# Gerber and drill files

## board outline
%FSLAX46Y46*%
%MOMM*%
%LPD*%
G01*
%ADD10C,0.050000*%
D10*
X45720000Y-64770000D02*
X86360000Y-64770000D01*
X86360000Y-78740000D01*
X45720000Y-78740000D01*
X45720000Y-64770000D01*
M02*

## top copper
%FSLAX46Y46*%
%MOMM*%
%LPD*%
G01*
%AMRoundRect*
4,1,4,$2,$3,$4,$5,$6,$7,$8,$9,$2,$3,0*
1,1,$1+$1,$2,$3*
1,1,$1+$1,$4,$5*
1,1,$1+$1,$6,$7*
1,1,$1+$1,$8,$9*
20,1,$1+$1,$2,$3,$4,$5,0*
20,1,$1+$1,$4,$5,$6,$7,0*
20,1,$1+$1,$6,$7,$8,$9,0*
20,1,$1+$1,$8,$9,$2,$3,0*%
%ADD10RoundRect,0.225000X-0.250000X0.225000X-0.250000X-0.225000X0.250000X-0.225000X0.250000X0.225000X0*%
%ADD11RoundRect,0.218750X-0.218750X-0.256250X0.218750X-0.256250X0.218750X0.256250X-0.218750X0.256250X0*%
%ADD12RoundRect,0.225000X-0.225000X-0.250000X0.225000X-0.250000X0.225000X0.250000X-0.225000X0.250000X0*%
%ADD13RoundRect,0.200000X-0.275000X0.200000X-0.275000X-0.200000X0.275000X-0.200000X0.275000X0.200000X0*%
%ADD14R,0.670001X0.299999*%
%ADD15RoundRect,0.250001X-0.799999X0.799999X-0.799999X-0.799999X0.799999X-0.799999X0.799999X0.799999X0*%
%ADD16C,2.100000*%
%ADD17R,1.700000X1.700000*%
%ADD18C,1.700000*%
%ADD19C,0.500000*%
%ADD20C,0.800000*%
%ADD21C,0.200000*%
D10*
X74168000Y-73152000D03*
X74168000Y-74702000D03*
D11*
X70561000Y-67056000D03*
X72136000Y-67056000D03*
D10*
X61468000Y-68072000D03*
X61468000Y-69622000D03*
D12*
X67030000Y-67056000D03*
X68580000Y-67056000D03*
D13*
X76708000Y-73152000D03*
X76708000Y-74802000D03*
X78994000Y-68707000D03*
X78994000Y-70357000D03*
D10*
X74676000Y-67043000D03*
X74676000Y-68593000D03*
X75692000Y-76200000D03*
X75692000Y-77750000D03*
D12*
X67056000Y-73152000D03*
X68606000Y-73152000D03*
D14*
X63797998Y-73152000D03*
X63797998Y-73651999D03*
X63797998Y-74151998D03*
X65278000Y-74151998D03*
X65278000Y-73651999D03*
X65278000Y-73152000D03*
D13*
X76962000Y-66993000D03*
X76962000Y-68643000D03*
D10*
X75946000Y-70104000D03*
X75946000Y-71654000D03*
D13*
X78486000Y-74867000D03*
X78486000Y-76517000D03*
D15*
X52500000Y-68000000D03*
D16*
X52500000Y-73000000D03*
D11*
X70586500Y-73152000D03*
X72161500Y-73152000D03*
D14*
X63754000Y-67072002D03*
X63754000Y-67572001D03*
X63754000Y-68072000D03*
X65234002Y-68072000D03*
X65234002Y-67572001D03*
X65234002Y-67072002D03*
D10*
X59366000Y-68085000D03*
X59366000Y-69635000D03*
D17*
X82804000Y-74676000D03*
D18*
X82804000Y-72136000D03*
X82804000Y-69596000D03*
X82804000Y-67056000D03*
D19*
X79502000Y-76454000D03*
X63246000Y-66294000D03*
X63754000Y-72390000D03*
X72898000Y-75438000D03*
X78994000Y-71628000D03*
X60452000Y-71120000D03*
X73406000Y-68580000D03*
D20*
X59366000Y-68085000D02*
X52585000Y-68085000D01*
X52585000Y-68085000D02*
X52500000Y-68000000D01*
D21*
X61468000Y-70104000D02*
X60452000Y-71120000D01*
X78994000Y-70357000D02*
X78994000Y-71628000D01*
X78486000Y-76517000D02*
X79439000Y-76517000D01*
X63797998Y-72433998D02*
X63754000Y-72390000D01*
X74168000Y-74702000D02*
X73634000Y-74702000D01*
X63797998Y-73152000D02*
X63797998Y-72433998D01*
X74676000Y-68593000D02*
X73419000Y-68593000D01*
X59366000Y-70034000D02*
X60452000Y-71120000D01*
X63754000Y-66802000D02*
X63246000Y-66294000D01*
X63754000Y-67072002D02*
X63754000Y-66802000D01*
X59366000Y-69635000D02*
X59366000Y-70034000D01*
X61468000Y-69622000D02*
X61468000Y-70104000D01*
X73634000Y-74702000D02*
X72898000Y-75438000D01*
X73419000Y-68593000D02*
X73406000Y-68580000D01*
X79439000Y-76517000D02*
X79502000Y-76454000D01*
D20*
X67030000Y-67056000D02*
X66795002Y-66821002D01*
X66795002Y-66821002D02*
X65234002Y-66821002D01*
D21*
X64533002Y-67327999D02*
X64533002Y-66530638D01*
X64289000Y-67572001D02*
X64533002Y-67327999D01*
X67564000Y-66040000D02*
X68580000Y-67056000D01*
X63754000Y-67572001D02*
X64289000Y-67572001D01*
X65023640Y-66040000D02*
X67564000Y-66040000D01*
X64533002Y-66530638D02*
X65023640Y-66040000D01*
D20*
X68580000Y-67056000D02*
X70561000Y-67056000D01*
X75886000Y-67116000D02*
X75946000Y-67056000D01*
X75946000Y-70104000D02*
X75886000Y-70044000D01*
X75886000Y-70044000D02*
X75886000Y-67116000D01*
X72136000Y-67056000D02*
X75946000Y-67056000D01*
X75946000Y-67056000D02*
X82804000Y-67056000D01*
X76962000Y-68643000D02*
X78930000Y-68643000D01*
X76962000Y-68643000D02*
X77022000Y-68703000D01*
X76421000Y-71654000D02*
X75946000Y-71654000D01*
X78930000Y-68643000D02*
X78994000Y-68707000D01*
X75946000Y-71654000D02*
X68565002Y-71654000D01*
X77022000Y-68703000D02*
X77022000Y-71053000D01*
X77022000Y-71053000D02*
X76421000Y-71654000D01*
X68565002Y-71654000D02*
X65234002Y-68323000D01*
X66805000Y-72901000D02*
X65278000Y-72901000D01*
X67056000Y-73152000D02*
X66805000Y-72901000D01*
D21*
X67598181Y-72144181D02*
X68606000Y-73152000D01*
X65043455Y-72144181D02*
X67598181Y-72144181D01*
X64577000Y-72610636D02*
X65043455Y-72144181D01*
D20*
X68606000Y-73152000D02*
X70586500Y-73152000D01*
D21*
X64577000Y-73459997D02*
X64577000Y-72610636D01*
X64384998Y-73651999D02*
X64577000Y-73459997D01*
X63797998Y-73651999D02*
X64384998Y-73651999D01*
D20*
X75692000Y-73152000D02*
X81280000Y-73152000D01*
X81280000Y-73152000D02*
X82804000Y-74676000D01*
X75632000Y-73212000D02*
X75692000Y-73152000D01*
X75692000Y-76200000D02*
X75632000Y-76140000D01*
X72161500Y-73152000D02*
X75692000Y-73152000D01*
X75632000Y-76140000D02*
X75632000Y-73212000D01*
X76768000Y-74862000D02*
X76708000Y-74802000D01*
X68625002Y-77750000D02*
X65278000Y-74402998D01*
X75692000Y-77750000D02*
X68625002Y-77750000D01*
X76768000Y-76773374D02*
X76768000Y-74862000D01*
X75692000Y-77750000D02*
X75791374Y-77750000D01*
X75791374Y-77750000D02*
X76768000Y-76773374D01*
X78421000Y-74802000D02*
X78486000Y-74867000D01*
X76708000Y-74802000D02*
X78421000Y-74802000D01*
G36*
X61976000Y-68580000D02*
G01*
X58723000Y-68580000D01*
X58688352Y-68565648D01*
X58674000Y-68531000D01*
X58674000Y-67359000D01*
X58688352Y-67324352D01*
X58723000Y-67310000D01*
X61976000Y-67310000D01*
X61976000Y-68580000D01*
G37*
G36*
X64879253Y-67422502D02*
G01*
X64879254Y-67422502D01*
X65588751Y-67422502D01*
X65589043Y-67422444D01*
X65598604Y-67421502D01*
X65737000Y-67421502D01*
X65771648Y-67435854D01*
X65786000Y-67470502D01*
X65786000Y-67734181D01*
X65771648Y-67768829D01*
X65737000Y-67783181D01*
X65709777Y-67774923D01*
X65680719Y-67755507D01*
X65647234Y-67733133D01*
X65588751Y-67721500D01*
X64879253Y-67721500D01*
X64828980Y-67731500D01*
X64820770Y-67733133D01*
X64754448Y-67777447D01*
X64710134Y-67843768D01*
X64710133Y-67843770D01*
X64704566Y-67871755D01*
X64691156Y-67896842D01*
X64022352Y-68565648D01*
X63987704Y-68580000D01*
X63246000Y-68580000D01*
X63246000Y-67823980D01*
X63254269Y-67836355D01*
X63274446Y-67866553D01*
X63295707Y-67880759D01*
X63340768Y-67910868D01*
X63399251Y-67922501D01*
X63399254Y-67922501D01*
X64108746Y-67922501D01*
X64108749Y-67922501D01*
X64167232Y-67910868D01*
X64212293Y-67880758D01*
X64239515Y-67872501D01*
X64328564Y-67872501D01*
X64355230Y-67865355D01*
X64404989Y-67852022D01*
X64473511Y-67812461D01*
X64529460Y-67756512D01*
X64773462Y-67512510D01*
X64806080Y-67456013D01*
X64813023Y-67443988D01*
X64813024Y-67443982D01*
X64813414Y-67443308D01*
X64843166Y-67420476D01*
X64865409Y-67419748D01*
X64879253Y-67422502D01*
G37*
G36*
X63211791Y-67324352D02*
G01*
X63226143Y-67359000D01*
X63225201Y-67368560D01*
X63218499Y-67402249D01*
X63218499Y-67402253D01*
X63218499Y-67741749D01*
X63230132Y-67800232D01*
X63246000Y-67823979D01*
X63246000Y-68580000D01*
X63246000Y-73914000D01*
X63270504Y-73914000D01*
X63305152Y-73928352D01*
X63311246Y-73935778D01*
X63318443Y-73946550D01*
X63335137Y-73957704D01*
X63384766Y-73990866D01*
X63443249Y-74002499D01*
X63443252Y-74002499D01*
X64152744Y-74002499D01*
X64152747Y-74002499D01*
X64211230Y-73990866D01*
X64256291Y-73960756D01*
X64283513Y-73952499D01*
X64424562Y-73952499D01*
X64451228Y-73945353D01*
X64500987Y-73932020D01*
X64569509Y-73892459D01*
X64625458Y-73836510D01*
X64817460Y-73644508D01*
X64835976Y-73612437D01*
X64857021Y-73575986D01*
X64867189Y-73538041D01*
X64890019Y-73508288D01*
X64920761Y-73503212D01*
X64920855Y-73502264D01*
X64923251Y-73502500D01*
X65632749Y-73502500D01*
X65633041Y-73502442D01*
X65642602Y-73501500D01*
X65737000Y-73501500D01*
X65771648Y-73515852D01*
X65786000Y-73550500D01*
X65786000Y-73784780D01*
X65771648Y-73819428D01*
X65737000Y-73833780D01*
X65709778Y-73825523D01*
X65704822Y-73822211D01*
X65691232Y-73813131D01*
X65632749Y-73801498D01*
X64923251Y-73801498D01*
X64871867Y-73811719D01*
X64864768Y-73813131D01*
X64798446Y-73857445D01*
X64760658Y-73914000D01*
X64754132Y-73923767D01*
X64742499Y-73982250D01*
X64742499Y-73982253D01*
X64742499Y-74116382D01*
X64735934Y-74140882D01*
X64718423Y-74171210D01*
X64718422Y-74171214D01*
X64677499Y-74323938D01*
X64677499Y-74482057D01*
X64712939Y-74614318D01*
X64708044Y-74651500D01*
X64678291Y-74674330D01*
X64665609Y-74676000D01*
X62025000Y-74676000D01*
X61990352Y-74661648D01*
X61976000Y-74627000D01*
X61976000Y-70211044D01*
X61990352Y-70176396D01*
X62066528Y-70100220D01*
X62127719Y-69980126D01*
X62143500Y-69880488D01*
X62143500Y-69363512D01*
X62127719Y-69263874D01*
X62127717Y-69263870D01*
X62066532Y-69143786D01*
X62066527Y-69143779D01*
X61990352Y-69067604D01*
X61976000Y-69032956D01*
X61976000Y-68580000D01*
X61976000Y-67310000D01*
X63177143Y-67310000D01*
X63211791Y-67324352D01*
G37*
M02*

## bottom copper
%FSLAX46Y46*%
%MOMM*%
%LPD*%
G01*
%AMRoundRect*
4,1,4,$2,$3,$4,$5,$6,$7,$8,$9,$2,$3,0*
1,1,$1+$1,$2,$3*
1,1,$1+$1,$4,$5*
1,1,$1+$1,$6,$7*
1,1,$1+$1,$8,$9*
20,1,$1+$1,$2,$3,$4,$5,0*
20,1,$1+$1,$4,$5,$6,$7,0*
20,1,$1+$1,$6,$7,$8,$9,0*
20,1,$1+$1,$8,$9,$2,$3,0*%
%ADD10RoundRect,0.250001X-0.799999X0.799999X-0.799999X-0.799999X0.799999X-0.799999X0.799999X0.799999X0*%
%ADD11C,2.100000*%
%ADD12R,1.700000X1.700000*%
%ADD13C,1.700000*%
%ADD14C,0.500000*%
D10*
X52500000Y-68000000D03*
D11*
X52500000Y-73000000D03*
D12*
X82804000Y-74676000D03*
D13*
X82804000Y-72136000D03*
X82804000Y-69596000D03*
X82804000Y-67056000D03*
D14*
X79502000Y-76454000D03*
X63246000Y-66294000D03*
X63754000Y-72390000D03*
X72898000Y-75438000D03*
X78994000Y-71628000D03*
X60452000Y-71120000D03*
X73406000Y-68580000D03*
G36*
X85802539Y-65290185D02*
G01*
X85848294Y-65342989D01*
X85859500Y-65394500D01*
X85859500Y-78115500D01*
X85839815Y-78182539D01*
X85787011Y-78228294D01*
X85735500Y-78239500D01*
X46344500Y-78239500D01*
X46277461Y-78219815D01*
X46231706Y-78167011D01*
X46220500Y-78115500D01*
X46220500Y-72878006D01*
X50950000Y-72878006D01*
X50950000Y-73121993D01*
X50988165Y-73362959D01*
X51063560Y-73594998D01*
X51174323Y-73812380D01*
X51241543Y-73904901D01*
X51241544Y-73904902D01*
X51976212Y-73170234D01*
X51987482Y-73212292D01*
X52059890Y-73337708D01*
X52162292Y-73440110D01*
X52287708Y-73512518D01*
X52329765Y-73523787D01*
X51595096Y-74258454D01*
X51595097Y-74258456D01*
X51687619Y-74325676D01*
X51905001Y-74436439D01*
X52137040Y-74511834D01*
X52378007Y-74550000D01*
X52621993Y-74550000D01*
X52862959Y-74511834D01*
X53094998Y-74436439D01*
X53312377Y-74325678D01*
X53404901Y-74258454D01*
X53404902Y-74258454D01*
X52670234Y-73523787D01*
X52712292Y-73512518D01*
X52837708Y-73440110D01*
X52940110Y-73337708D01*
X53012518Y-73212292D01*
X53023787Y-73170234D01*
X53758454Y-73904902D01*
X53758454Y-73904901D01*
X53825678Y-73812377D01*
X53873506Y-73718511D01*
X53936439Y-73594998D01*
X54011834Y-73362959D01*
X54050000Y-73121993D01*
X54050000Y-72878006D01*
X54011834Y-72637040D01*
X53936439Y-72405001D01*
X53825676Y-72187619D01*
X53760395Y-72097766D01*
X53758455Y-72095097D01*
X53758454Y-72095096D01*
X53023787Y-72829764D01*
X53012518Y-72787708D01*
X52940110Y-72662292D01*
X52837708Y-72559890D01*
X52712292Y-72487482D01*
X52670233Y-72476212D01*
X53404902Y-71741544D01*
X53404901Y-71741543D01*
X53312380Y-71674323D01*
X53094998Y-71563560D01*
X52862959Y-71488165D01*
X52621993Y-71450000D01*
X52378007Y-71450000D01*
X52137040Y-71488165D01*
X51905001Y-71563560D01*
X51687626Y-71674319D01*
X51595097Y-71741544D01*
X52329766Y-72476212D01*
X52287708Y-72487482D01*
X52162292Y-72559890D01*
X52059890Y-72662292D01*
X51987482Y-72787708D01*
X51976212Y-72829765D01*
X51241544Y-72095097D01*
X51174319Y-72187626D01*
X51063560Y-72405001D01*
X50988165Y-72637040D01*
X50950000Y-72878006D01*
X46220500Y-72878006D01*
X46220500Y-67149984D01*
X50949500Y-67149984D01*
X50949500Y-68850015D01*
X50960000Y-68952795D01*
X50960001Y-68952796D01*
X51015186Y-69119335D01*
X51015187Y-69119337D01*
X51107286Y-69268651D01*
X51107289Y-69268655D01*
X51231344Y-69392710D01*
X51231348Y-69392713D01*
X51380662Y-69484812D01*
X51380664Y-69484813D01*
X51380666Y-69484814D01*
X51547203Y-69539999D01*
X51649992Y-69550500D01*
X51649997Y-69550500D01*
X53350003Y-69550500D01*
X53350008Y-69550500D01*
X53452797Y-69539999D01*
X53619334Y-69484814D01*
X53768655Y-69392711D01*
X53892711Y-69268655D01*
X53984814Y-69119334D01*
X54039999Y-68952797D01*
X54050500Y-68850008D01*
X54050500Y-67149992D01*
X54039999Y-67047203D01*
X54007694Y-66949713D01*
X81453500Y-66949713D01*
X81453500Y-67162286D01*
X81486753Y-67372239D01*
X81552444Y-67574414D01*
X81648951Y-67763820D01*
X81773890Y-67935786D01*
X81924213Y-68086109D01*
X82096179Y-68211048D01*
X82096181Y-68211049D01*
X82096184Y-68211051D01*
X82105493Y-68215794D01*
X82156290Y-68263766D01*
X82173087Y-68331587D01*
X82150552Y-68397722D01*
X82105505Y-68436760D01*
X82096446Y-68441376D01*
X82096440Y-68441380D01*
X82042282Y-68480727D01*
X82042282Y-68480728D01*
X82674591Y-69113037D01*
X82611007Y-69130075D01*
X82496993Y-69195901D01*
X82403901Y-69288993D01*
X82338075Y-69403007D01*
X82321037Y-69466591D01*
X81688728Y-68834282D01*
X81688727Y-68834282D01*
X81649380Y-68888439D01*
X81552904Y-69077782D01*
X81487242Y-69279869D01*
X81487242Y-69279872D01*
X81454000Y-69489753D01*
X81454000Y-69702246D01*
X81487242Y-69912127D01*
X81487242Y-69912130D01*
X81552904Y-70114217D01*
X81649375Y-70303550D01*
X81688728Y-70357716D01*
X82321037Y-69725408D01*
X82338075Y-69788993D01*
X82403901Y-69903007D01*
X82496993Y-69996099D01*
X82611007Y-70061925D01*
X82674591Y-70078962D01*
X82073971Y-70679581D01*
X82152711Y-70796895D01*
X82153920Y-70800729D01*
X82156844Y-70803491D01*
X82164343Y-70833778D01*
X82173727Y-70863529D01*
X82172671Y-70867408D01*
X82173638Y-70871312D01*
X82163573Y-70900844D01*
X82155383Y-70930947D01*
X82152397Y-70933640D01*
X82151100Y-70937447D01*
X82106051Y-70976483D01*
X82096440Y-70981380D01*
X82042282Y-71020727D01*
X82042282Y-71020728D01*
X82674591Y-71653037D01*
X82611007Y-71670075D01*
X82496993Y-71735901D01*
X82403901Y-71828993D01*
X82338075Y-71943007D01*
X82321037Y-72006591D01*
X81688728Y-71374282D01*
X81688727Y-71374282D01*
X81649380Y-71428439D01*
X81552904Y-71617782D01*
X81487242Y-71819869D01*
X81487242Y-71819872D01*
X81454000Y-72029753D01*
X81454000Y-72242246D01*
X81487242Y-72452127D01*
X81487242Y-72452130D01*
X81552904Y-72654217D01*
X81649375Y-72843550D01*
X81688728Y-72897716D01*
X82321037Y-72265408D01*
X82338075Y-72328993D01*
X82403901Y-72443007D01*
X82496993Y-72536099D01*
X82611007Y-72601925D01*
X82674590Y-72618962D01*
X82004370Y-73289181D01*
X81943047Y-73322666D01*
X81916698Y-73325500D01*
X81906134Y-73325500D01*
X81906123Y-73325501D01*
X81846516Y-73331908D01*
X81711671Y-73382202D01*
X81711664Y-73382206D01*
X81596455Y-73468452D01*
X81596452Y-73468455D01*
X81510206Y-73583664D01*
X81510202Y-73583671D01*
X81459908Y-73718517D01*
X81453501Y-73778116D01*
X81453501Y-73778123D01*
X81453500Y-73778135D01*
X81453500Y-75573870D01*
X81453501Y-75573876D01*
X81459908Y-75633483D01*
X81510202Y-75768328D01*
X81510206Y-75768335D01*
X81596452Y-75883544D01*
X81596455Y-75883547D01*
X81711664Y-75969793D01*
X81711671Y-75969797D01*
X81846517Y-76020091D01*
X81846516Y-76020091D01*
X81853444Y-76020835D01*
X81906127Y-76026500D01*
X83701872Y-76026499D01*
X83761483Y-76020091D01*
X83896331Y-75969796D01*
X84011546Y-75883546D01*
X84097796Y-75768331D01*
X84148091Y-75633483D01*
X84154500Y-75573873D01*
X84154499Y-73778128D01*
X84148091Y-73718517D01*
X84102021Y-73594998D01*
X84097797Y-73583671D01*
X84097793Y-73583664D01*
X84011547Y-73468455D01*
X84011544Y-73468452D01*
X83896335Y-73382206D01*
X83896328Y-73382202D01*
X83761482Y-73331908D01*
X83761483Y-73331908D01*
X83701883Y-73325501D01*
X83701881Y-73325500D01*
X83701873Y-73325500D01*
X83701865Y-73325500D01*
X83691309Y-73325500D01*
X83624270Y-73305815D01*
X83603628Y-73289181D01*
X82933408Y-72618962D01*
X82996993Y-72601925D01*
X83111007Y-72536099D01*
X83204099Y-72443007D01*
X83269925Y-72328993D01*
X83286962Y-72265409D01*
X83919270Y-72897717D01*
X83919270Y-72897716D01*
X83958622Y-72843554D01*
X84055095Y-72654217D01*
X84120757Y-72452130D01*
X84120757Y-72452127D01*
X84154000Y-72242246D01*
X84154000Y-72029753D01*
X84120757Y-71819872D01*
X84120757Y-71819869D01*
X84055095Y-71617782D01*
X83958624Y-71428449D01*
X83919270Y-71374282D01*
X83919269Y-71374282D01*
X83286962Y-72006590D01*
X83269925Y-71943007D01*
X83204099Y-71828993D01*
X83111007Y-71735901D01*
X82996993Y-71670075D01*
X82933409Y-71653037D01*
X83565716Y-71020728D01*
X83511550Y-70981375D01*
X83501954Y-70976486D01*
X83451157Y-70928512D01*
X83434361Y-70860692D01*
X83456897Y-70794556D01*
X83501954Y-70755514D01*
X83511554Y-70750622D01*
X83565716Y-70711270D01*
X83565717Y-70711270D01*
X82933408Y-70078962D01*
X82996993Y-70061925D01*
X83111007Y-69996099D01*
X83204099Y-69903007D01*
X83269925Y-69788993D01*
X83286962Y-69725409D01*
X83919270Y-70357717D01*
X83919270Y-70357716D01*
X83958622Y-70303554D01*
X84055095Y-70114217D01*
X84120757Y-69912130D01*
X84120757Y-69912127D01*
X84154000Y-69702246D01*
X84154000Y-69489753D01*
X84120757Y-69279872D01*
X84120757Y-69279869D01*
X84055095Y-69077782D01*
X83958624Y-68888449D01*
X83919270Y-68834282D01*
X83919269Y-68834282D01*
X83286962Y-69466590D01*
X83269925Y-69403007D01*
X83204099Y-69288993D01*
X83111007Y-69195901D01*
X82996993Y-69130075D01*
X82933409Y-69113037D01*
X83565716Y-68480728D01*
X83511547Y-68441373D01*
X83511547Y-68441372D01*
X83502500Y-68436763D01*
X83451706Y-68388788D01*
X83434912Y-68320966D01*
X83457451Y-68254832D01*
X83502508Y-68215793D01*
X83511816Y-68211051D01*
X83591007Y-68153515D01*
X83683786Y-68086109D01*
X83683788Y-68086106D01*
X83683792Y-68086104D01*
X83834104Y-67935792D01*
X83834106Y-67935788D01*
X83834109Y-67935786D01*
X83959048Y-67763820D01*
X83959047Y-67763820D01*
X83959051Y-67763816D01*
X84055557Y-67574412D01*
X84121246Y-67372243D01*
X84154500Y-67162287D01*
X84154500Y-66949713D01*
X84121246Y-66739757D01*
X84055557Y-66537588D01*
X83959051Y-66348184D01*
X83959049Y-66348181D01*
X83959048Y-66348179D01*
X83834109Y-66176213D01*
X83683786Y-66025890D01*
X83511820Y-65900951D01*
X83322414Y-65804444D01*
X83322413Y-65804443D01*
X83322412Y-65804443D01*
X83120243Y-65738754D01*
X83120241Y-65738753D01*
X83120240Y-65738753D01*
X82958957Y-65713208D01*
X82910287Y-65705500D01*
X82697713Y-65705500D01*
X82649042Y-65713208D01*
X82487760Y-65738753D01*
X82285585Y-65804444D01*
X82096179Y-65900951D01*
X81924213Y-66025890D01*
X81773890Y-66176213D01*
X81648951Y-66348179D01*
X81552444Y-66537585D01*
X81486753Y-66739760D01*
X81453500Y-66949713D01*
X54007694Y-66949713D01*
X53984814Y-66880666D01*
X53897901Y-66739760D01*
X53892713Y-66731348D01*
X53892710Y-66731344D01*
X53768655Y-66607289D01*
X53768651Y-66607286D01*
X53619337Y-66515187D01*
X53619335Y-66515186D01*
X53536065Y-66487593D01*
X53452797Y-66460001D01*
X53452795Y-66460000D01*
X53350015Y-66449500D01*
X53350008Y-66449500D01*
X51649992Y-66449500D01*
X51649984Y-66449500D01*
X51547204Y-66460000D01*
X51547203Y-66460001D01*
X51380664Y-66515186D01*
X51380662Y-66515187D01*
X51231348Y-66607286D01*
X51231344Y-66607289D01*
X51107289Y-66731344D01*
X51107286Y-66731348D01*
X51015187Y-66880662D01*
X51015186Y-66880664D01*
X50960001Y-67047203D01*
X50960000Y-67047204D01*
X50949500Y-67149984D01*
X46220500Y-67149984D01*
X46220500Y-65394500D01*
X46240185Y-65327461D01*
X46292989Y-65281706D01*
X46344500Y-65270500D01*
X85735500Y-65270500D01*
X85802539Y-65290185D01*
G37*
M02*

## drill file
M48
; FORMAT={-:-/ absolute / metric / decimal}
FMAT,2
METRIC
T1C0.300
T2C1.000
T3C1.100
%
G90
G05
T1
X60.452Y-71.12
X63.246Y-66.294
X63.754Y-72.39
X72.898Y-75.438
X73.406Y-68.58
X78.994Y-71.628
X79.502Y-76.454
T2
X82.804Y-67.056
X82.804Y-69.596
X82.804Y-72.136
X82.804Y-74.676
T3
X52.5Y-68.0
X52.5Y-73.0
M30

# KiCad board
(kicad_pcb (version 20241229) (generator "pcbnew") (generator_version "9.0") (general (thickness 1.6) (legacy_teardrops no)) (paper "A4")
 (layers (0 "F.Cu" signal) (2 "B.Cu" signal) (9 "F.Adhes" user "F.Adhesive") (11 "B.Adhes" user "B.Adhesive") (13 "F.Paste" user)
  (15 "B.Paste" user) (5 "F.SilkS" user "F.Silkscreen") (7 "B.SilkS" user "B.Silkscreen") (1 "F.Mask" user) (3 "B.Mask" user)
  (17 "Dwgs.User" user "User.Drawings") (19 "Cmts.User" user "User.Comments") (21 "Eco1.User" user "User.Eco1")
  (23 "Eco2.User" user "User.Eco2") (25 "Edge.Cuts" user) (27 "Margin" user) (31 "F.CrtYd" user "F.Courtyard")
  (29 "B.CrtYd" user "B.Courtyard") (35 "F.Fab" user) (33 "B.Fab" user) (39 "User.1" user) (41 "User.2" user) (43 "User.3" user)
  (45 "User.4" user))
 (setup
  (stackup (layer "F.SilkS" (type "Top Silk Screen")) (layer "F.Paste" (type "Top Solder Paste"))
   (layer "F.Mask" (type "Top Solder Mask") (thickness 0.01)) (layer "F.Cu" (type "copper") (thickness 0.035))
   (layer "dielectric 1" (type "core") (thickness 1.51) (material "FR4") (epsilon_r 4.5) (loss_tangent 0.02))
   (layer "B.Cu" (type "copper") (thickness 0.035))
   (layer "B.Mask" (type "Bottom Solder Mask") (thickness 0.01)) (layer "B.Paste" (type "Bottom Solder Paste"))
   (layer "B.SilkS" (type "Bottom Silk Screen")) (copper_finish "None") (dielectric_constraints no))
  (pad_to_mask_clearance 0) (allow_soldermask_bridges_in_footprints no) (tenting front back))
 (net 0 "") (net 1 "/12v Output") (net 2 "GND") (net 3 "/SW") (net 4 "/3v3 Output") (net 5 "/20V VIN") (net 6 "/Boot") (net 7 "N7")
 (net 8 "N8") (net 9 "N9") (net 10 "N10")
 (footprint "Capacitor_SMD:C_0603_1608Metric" (layer "F.Cu") (at 74.168 73.927 -90)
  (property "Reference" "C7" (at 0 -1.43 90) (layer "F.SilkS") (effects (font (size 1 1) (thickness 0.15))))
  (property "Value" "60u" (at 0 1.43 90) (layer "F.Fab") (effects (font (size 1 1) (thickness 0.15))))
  (pad "1" smd roundrect (at -0.775 0 270) (size 0.9 0.95) (layers "F.Cu" "F.Mask" "F.Paste") (roundrect_rratio 0.25) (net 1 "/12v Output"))
  (pad "2" smd roundrect (at 0.775 0 270) (size 0.9 0.95) (layers "F.Cu" "F.Mask" "F.Paste") (roundrect_rratio 0.25) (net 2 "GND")))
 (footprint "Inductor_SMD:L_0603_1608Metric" (layer "F.Cu") (at 71.3485 67.056)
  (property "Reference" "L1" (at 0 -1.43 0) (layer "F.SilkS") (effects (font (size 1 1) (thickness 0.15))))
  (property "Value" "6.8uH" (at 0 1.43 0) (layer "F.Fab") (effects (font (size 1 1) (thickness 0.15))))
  (pad "1" smd roundrect (at -0.7875 0) (size 0.875 0.95) (layers "F.Cu" "F.Mask" "F.Paste") (roundrect_rratio 0.25) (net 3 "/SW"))
  (pad "2" smd roundrect (at 0.7875 0) (size 0.875 0.95) (layers "F.Cu" "F.Mask" "F.Paste") (roundrect_rratio 0.25) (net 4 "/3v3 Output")))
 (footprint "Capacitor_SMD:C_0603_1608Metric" (layer "F.Cu") (at 61.468 68.847 -90)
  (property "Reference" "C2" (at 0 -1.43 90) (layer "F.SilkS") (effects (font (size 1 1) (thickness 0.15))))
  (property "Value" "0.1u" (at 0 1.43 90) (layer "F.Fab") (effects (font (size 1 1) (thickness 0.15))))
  (pad "1" smd roundrect (at -0.775 0 270) (size 0.9 0.95) (layers "F.Cu" "F.Mask" "F.Paste") (roundrect_rratio 0.25) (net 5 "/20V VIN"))
  (pad "2" smd roundrect (at 0.775 0 270) (size 0.9 0.95) (layers "F.Cu" "F.Mask" "F.Paste") (roundrect_rratio 0.25) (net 2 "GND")))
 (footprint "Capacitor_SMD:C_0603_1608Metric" (layer "F.Cu") (at 67.805 67.056)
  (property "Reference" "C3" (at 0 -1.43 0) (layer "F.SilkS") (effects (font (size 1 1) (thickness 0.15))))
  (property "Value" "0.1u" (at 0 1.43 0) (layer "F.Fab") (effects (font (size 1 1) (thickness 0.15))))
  (pad "1" smd roundrect (at -0.775 0) (size 0.9 0.95) (layers "F.Cu" "F.Mask" "F.Paste") (roundrect_rratio 0.25) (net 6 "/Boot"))
  (pad "2" smd roundrect (at 0.775 0) (size 0.9 0.95) (layers "F.Cu" "F.Mask" "F.Paste") (roundrect_rratio 0.25) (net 3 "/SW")))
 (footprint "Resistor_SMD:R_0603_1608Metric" (layer "F.Cu") (at 76.708 73.977 -90)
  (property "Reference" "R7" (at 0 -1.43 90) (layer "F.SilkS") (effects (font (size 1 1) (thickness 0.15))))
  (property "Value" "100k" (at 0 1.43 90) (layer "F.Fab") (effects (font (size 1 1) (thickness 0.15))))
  (pad "1" smd roundrect (at -0.825 0 270) (size 0.8 0.95) (layers "F.Cu" "F.Mask" "F.Paste") (roundrect_rratio 0.25) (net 1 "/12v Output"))
  (pad "2" smd roundrect (at 0.825 0 270) (size 0.8 0.95) (layers "F.Cu" "F.Mask" "F.Paste") (roundrect_rratio 0.25) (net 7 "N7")))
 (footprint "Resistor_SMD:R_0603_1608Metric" (layer "F.Cu") (at 78.994 69.532 -90)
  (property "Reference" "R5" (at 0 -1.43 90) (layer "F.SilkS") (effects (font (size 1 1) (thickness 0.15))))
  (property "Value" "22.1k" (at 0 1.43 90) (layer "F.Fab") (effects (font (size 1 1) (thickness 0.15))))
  (pad "1" smd roundrect (at -0.825 0 270) (size 0.8 0.95) (layers "F.Cu" "F.Mask" "F.Paste") (roundrect_rratio 0.25) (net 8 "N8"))
  (pad "2" smd roundrect (at 0.825 0 270) (size 0.8 0.95) (layers "F.Cu" "F.Mask" "F.Paste") (roundrect_rratio 0.25) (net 2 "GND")))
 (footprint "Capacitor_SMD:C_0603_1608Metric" (layer "F.Cu") (at 74.676 67.818 -90)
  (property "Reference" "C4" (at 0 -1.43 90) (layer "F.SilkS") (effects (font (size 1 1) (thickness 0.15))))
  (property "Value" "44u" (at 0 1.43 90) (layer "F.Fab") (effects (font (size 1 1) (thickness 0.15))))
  (pad "1" smd roundrect (at -0.775 0 270) (size 0.9 0.95) (layers "F.Cu" "F.Mask" "F.Paste") (roundrect_rratio 0.25) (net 4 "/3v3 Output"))
  (pad "2" smd roundrect (at 0.775 0 270) (size 0.9 0.95) (layers "F.Cu" "F.Mask" "F.Paste") (roundrect_rratio 0.25) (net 2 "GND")))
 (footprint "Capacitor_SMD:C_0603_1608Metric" (layer "F.Cu") (at 75.692 76.975 -90)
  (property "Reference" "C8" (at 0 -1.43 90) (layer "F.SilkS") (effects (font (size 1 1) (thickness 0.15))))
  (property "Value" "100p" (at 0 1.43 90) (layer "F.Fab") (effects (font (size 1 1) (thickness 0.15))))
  (pad "1" smd roundrect (at -0.775 0 270) (size 0.9 0.95) (layers "F.Cu" "F.Mask" "F.Paste") (roundrect_rratio 0.25) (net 1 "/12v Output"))
  (pad "2" smd roundrect (at 0.775 0 270) (size 0.9 0.95) (layers "F.Cu" "F.Mask" "F.Paste") (roundrect_rratio 0.25) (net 7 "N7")))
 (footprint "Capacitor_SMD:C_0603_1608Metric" (layer "F.Cu") (at 67.831 73.152)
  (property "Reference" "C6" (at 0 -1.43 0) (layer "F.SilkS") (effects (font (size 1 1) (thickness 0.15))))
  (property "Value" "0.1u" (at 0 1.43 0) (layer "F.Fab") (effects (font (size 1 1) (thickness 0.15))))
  (pad "1" smd roundrect (at -0.775 0) (size 0.9 0.95) (layers "F.Cu" "F.Mask" "F.Paste") (roundrect_rratio 0.25) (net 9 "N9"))
  (pad "2" smd roundrect (at 0.775 0) (size 0.9 0.95) (layers "F.Cu" "F.Mask" "F.Paste") (roundrect_rratio 0.25) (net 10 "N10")))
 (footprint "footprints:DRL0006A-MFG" (layer "F.Cu") (at 64.537999 73.651999)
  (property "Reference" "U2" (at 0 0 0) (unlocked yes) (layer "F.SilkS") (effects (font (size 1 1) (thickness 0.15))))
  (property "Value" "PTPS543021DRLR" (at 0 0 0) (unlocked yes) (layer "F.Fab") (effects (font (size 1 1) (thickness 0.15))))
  (pad "1" smd rect (at -0.740001 -0.499999) (size 0.670001 0.299999) (layers "F.Cu" "F.Mask" "F.Paste") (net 2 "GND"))
  (pad "2" smd rect (at -0.740001 0) (size 0.670001 0.299999) (layers "F.Cu" "F.Mask" "F.Paste") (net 10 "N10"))
  (pad "3" smd rect (at -0.740001 0.499999) (size 0.670001 0.299999) (layers "F.Cu" "F.Mask" "F.Paste") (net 5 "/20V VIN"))
  (pad "4" smd rect (at 0.740001 0.499999) (size 0.670001 0.299999) (layers "F.Cu" "F.Mask" "F.Paste") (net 7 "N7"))
  (pad "5" smd rect (at 0.740001 0) (size 0.670001 0.299999) (layers "F.Cu" "F.Mask" "F.Paste") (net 5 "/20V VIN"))
  (pad "6" smd rect (at 0.740001 -0.499999) (size 0.670001 0.299999) (layers "F.Cu" "F.Mask" "F.Paste") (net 9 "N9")))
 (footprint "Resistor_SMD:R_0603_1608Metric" (layer "F.Cu") (at 76.962 67.818 -90)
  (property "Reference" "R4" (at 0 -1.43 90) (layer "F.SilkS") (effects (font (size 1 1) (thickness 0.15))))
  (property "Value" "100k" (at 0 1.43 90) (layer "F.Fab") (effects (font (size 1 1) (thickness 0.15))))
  (pad "1" smd roundrect (at -0.825 0 270) (size 0.8 0.95) (layers "F.Cu" "F.Mask" "F.Paste") (roundrect_rratio 0.25) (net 4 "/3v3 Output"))
  (pad "2" smd roundrect (at 0.825 0 270) (size 0.8 0.95) (layers "F.Cu" "F.Mask" "F.Paste") (roundrect_rratio 0.25) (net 8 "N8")))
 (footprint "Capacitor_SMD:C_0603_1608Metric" (layer "F.Cu") (at 75.946 70.879 -90)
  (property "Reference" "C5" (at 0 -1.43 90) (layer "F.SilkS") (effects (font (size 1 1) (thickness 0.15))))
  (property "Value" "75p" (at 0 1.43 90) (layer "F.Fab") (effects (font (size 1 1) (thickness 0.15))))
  (pad "1" smd roundrect (at -0.775 0 270) (size 0.9 0.95) (layers "F.Cu" "F.Mask" "F.Paste") (roundrect_rratio 0.25) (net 4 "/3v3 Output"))
  (pad "2" smd roundrect (at 0.775 0 270) (size 0.9 0.95) (layers "F.Cu" "F.Mask" "F.Paste") (roundrect_rratio 0.25) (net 8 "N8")))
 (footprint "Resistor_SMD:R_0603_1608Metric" (layer "F.Cu") (at 78.486 75.692 -90)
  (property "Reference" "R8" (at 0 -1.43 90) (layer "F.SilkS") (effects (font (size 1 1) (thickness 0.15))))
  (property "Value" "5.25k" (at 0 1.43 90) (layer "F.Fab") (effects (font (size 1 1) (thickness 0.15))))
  (pad "1" smd roundrect (at -0.825 0 270) (size 0.8 0.95) (layers "F.Cu" "F.Mask" "F.Paste") (roundrect_rratio 0.25) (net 7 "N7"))
  (pad "2" smd roundrect (at 0.825 0 270) (size 0.8 0.95) (layers "F.Cu" "F.Mask" "F.Paste") (roundrect_rratio 0.25) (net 2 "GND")))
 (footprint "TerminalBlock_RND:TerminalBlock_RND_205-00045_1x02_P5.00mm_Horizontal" (layer "F.Cu") (at 52.5 68 -90)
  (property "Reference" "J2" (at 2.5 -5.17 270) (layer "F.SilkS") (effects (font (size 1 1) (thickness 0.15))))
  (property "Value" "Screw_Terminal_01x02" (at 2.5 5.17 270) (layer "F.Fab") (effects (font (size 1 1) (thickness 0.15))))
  (pad "1" thru_hole roundrect (at 0 0 270) (size 2.1 2.1) (drill 1.1) (layers "*.Cu" "*.Mask") (remove_unused_layers no)
   (roundrect_rratio 0.119048) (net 5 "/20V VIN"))
  (pad "2" thru_hole circle (at 5 0 270) (size 2.1 2.1) (drill 1.1) (layers "*.Cu" "*.Mask") (remove_unused_layers no) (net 2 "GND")))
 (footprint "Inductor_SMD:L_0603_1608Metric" (layer "F.Cu") (at 71.374 73.152)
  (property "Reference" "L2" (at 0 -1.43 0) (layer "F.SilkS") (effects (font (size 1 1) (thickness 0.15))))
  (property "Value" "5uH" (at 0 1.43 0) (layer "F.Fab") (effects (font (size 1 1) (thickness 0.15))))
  (pad "1" smd roundrect (at -0.7875 0) (size 0.875 0.95) (layers "F.Cu" "F.Mask" "F.Paste") (roundrect_rratio 0.25) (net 10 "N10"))
  (pad "2" smd roundrect (at 0.7875 0) (size 0.875 0.95) (layers "F.Cu" "F.Mask" "F.Paste") (roundrect_rratio 0.25) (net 1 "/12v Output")))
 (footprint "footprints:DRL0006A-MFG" (layer "F.Cu") (at 64.494001 67.572001)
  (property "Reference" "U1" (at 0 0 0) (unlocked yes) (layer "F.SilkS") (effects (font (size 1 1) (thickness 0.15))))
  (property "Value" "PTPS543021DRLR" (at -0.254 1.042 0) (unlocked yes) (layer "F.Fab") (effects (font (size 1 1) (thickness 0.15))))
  (pad "1" smd rect (at -0.740001 -0.499999) (size 0.670001 0.299999) (layers "F.Cu" "F.Mask" "F.Paste") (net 2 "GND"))
  (pad "2" smd rect (at -0.740001 0) (size 0.670001 0.299999) (layers "F.Cu" "F.Mask" "F.Paste") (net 3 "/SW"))
  (pad "3" smd rect (at -0.740001 0.499999) (size 0.670001 0.299999) (layers "F.Cu" "F.Mask" "F.Paste") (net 5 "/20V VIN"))
  (pad "4" smd rect (at 0.740001 0.499999) (size 0.670001 0.299999) (layers "F.Cu" "F.Mask" "F.Paste") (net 8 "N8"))
  (pad "5" smd rect (at 0.740001 0) (size 0.670001 0.299999) (layers "F.Cu" "F.Mask" "F.Paste") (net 5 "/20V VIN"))
  (pad "6" smd rect (at 0.740001 -0.499999) (size 0.670001 0.299999) (layers "F.Cu" "F.Mask" "F.Paste") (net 6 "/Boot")))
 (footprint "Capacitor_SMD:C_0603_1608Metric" (layer "F.Cu") (at 59.366 68.86 -90)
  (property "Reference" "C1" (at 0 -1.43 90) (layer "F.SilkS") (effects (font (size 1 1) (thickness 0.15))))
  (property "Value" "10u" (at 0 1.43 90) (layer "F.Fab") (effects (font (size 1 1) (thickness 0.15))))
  (pad "1" smd roundrect (at -0.775 0 270) (size 0.9 0.95) (layers "F.Cu" "F.Mask" "F.Paste") (roundrect_rratio 0.25) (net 5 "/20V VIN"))
  (pad "2" smd roundrect (at 0.775 0 270) (size 0.9 0.95) (layers "F.Cu" "F.Mask" "F.Paste") (roundrect_rratio 0.25) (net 2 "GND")))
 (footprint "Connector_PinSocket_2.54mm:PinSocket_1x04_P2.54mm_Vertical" (layer "B.Cu") (at 82.804 74.676)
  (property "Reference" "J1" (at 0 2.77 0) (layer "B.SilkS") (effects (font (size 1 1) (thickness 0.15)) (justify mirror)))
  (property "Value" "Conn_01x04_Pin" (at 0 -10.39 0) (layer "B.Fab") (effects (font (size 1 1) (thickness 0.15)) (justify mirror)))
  (pad "1" thru_hole rect (at 0 0) (size 1.7 1.7) (drill 1) (layers "*.Cu" "*.Mask") (remove_unused_layers no) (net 1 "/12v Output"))
  (pad "2" thru_hole circle (at 0 -2.54) (size 1.7 1.7) (drill 1) (layers "*.Cu" "*.Mask") (remove_unused_layers no) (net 2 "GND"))
  (pad "3" thru_hole circle (at 0 -5.08) (size 1.7 1.7) (drill 1) (layers "*.Cu" "*.Mask") (remove_unused_layers no) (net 2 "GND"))
  (pad "4" thru_hole circle (at 0 -7.62) (size 1.7 1.7) (drill 1) (layers "*.Cu" "*.Mask") (remove_unused_layers no) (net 4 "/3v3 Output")))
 (gr_rect (start 45.72 64.77) (end 86.36 78.74) (stroke (width 0.05) (type default)) (fill no) (layer "Edge.Cuts"))
 (segment (start 59.366 68.085) (end 52.585 68.085) (width 0.8) (layer "F.Cu") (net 5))
 (segment (start 52.585 68.085) (end 52.5 68) (width 0.8) (layer "F.Cu") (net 5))
 (segment (start 61.468 70.104) (end 60.452 71.12) (width 0.2) (layer "F.Cu") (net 2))
 (segment (start 78.994 70.357) (end 78.994 71.628) (width 0.2) (layer "F.Cu") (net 2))
 (segment (start 78.486 76.517) (end 79.439 76.517) (width 0.2) (layer "F.Cu") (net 2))
 (segment (start 63.797998 72.433998) (end 63.754 72.39) (width 0.2) (layer "F.Cu") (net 2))
 (segment (start 74.168 74.702) (end 73.634 74.702) (width 0.2) (layer "F.Cu") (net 2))
 (segment (start 63.797998 73.152) (end 63.797998 72.433998) (width 0.2) (layer "F.Cu") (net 2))
 (segment (start 74.676 68.593) (end 73.419 68.593) (width 0.2) (layer "F.Cu") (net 2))
 (segment (start 59.366 70.034) (end 60.452 71.12) (width 0.2) (layer "F.Cu") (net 2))
 (segment (start 63.754 66.802) (end 63.246 66.294) (width 0.2) (layer "F.Cu") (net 2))
 (segment (start 63.754 67.072002) (end 63.754 66.802) (width 0.2) (layer "F.Cu") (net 2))
 (segment (start 59.366 69.635) (end 59.366 70.034) (width 0.2) (layer "F.Cu") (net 2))
 (segment (start 61.468 69.622) (end 61.468 70.104) (width 0.2) (layer "F.Cu") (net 2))
 (segment (start 73.634 74.702) (end 72.898 75.438) (width 0.2) (layer "F.Cu") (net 2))
 (segment (start 73.419 68.593) (end 73.406 68.58) (width 0.2) (layer "F.Cu") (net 2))
 (segment (start 79.439 76.517) (end 79.502 76.454) (width 0.2) (layer "F.Cu") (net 2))
 (via (at 79.502 76.454) (size 0.5) (drill 0.3) (layers "F.Cu" "B.Cu") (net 2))
 (via (at 63.246 66.294) (size 0.5) (drill 0.3) (layers "F.Cu" "B.Cu") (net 2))
 (via (at 63.754 72.39) (size 0.5) (drill 0.3) (layers "F.Cu" "B.Cu") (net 2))
 (via (at 72.898 75.438) (size 0.5) (drill 0.3) (layers "F.Cu" "B.Cu") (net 2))
 (via (at 78.994 71.628) (size 0.5) (drill 0.3) (layers "F.Cu" "B.Cu") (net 2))
 (via (at 60.452 71.12) (size 0.5) (drill 0.3) (layers "F.Cu" "B.Cu") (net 2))
 (via (at 73.406 68.58) (size 0.5) (drill 0.3) (layers "F.Cu" "B.Cu") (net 2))
 (segment (start 67.03 67.056) (end 66.795002 66.821002) (width 0.8) (layer "F.Cu") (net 6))
 (segment (start 66.795002 66.821002) (end 65.234002 66.821002) (width 0.8) (layer "F.Cu") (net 6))
 (segment (start 64.533002 67.327999) (end 64.533002 66.530638) (width 0.2) (layer "F.Cu") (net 3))
 (segment (start 64.289 67.572001) (end 64.533002 67.327999) (width 0.2) (layer "F.Cu") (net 3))
 (segment (start 67.564 66.04) (end 68.58 67.056) (width 0.2) (layer "F.Cu") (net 3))
 (segment (start 63.754 67.572001) (end 64.289 67.572001) (width 0.2) (layer "F.Cu") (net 3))
 (segment (start 65.02364 66.04) (end 67.564 66.04) (width 0.2) (layer "F.Cu") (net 3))
 (segment (start 64.533002 66.530638) (end 65.02364 66.04) (width 0.2) (layer "F.Cu") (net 3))
 (segment (start 68.58 67.056) (end 70.561 67.056) (width 0.8) (layer "F.Cu") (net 3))
 (segment (start 75.886 67.116) (end 75.946 67.056) (width 0.8) (layer "F.Cu") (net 4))
 (segment (start 75.946 70.104) (end 75.886 70.044) (width 0.8) (layer "F.Cu") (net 4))
 (segment (start 75.886 70.044) (end 75.886 67.116) (width 0.8) (layer "F.Cu") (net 4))
 (segment (start 72.136 67.056) (end 75.946 67.056) (width 0.8) (layer "F.Cu") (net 4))
 (segment (start 75.946 67.056) (end 82.804 67.056) (width 0.8) (layer "F.Cu") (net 4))
 (segment (start 76.962 68.643) (end 78.93 68.643) (width 0.8) (layer "F.Cu") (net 8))
 (segment (start 76.962 68.643) (end 77.022 68.703) (width 0.8) (layer "F.Cu") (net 8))
 (segment (start 76.421 71.654) (end 75.946 71.654) (width 0.8) (layer "F.Cu") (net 8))
 (segment (start 78.93 68.643) (end 78.994 68.707) (width 0.8) (layer "F.Cu") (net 8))
 (segment (start 75.946 71.654) (end 68.565002 71.654) (width 0.8) (layer "F.Cu") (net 8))
 (segment (start 77.022 68.703) (end 77.022 71.053) (width 0.8) (layer "F.Cu") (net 8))
 (segment (start 77.022 71.053) (end 76.421 71.654) (width 0.8) (layer "F.Cu") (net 8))
 (segment (start 68.565002 71.654) (end 65.234002 68.323) (width 0.8) (layer "F.Cu") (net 8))
 (segment (start 66.805 72.901) (end 65.278 72.901) (width 0.8) (layer "F.Cu") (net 9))
 (segment (start 67.056 73.152) (end 66.805 72.901) (width 0.8) (layer "F.Cu") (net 9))
 (segment (start 67.598181 72.144181) (end 68.606 73.152) (width 0.2) (layer "F.Cu") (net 10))
 (segment (start 65.043455 72.144181) (end 67.598181 72.144181) (width 0.2) (layer "F.Cu") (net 10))
 (segment (start 64.577 72.610636) (end 65.043455 72.144181) (width 0.2) (layer "F.Cu") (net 10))
 (segment (start 68.606 73.152) (end 70.5865 73.152) (width 0.8) (layer "F.Cu") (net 10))
 (segment (start 64.577 73.459997) (end 64.577 72.610636) (width 0.2) (layer "F.Cu") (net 10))
 (segment (start 64.384998 73.651999) (end 64.577 73.459997) (width 0.2) (layer "F.Cu") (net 10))
 (segment (start 63.797998 73.651999) (end 64.384998 73.651999) (width 0.2) (layer "F.Cu") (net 10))
 (segment (start 75.692 73.152) (end 81.28 73.152) (width 0.8) (layer "F.Cu") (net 1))
 (segment (start 81.28 73.152) (end 82.804 74.676) (width 0.8) (layer "F.Cu") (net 1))
 (segment (start 75.632 73.212) (end 75.692 73.152) (width 0.8) (layer "F.Cu") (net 1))
 (segment (start 75.692 76.2) (end 75.632 76.14) (width 0.8) (layer "F.Cu") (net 1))
 (segment (start 72.1615 73.152) (end 75.692 73.152) (width 0.8) (layer "F.Cu") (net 1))
 (segment (start 75.632 76.14) (end 75.632 73.212) (width 0.8) (layer "F.Cu") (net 1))
 (segment (start 76.768 74.862) (end 76.708 74.802) (width 0.8) (layer "F.Cu") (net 7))
 (segment (start 68.625002 77.75) (end 65.278 74.402998) (width 0.8) (layer "F.Cu") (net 7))
 (segment (start 75.692 77.75) (end 68.625002 77.75) (width 0.8) (layer "F.Cu") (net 7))
 (segment (start 76.768 76.773374) (end 76.768 74.862) (width 0.8) (layer "F.Cu") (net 7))
 (segment (start 75.692 77.75) (end 75.791374 77.75) (width 0.8) (layer "F.Cu") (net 7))
 (segment (start 75.791374 77.75) (end 76.768 76.773374) (width 0.8) (layer "F.Cu") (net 7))
 (segment (start 78.421 74.802) (end 78.486 74.867) (width 0.8) (layer "F.Cu") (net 7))
 (segment (start 76.708 74.802) (end 78.421 74.802) (width 0.8) (layer "F.Cu") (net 7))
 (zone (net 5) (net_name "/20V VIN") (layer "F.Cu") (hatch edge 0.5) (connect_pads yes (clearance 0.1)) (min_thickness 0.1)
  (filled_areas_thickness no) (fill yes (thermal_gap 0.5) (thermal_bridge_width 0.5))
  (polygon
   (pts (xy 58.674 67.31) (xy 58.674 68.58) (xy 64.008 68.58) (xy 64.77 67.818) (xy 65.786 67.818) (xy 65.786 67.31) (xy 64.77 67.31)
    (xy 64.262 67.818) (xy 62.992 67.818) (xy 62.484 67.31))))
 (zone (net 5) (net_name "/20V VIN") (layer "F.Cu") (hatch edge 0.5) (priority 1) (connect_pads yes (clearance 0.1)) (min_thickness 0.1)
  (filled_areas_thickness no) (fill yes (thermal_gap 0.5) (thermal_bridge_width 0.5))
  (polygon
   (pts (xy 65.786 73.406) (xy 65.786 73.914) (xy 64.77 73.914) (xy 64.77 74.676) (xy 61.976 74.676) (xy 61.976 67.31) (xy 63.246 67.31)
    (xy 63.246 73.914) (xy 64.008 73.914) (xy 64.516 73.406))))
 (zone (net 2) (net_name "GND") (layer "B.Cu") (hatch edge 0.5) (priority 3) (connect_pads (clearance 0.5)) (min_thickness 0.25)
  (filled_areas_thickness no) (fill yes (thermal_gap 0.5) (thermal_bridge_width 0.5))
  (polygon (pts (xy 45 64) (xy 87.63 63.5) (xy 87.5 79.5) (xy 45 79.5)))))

